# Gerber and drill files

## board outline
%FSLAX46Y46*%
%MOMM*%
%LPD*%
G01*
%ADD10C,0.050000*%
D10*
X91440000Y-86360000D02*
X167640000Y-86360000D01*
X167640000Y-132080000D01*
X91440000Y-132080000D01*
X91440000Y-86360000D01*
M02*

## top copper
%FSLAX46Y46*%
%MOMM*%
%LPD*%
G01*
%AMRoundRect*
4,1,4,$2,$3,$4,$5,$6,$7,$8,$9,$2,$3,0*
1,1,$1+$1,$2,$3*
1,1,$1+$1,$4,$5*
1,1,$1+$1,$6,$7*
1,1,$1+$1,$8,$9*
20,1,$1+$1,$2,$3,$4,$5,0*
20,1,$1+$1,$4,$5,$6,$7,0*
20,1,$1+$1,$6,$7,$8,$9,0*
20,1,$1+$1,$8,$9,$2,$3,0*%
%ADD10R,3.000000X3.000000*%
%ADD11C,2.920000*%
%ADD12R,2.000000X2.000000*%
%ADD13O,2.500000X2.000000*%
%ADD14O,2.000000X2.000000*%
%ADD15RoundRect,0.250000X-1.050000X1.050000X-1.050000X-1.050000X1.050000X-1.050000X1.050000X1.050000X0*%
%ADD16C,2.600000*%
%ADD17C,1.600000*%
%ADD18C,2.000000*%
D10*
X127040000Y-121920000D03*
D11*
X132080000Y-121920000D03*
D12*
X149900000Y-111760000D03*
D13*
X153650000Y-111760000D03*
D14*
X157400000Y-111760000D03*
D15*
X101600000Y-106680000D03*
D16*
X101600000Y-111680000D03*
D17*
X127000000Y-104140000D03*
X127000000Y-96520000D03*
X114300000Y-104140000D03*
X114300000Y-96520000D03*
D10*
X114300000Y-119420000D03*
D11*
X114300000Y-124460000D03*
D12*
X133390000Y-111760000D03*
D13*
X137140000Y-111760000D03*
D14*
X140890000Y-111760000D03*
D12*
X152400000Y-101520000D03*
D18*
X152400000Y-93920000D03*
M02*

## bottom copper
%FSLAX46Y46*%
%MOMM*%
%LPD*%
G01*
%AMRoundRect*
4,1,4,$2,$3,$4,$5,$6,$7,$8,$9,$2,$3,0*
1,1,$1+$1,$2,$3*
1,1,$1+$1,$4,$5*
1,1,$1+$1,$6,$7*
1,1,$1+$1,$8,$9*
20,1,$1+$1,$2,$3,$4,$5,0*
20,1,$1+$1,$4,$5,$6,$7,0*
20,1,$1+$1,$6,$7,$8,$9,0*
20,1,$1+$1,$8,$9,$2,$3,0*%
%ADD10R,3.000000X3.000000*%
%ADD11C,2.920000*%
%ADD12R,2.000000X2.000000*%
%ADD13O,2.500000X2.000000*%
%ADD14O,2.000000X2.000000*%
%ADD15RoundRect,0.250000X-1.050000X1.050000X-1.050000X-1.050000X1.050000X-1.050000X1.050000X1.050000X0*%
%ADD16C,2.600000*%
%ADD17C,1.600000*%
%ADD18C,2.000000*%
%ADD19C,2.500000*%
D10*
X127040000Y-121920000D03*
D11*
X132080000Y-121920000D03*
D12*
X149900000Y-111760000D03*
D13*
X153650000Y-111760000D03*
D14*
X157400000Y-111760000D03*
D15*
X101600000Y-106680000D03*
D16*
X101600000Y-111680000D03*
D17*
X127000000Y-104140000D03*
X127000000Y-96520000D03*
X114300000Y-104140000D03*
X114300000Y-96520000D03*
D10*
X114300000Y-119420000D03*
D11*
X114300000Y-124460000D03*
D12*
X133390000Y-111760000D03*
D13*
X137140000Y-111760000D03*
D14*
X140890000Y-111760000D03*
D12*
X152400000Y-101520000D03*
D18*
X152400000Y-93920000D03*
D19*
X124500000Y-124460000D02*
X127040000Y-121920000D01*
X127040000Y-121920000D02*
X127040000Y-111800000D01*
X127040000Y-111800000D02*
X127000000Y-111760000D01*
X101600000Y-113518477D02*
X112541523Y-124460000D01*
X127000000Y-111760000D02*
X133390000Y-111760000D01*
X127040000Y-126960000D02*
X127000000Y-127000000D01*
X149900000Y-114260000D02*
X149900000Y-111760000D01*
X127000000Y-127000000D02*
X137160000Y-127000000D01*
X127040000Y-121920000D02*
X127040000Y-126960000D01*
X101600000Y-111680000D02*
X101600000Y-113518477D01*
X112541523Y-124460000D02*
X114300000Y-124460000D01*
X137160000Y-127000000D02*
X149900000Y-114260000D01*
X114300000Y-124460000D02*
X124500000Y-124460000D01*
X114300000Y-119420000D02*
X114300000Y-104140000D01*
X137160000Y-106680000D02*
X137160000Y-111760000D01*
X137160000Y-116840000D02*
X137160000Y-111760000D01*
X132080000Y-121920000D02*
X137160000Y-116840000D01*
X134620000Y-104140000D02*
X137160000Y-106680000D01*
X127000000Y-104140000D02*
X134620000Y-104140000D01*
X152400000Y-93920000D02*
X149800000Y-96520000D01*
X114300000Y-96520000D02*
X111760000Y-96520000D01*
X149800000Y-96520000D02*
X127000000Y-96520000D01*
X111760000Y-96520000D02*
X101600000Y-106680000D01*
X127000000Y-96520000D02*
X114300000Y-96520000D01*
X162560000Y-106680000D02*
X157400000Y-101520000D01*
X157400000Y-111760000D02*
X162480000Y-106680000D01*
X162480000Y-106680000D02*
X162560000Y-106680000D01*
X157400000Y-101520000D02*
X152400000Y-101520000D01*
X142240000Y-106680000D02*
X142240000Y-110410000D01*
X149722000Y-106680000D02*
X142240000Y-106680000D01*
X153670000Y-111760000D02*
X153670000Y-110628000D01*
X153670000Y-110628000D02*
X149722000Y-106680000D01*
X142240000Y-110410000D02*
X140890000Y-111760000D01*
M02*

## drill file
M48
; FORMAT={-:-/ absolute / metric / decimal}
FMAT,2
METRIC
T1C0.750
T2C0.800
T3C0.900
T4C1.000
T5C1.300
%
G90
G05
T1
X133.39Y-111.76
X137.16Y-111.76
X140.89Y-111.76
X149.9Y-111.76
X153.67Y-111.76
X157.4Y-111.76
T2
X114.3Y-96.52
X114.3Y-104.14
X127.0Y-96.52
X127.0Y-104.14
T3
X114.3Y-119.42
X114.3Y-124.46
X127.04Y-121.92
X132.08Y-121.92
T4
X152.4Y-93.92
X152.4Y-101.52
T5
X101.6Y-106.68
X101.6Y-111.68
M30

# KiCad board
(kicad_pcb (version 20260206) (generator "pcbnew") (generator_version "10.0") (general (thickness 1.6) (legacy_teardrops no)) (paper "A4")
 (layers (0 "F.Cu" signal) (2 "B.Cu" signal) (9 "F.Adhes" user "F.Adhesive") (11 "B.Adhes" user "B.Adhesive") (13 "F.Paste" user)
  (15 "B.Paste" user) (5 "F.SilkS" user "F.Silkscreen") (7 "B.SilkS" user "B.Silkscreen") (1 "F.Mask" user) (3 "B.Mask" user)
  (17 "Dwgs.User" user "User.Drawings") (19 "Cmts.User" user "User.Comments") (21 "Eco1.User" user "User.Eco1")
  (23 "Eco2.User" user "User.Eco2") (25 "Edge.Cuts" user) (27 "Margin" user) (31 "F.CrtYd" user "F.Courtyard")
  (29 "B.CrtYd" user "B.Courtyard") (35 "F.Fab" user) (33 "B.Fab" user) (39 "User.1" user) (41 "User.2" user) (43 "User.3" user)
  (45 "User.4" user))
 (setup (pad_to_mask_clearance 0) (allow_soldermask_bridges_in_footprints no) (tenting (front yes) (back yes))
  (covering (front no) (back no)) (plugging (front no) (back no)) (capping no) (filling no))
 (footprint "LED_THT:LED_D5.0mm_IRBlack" (layer "F.Cu") (at 129.54 121.92)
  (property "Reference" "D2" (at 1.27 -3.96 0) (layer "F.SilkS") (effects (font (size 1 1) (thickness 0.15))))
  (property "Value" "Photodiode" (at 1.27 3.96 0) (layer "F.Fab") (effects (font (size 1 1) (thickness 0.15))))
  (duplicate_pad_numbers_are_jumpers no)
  (pad "1" thru_hole rect (at -2.5 0) (size 3 3) (drill 0.9) (layers "*.Cu" "*.Mask") (remove_unused_layers no) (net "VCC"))
  (pad "2" thru_hole circle (at 2.54 0) (size 2.92 2.92) (drill 0.9) (layers "*.Cu" "*.Mask") (remove_unused_layers no) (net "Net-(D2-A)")))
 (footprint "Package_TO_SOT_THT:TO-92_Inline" (layer "F.Cu") (at 152.4 111.76)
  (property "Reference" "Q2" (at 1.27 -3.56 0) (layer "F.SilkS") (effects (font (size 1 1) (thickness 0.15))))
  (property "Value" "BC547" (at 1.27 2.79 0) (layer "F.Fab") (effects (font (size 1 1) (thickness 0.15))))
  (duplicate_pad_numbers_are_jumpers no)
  (pad "1" thru_hole rect (at -2.5 0) (size 2 2) (drill 0.75) (layers "*.Cu" "*.Mask") (remove_unused_layers no) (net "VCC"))
  (pad "2" thru_hole oval (at 1.27 0) (size 2.5 2) (drill 0.75 (offset -0.02 0)) (layers "*.Cu" "*.Mask") (remove_unused_layers no)
   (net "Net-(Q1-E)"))
  (pad "3" thru_hole oval (at 5 0) (size 2 2) (drill 0.75) (layers "*.Cu" "*.Mask") (remove_unused_layers no) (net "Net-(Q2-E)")))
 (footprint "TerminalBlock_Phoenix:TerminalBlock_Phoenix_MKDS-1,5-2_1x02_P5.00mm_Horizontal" (layer "F.Cu") (at 101.6 106.68 -90)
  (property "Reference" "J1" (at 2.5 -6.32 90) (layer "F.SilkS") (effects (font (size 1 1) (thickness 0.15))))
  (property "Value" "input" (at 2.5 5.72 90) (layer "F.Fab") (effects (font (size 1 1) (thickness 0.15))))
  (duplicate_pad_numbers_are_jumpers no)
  (pad "1" thru_hole roundrect (at 0 0 270) (size 2.6 2.6) (drill 1.3) (layers "*.Cu" "*.Mask") (remove_unused_layers no)
   (roundrect_rratio 0.096154) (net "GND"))
  (pad "2" thru_hole circle (at 5 0 270) (size 2.6 2.6) (drill 1.3) (layers "*.Cu" "*.Mask") (remove_unused_layers no) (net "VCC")))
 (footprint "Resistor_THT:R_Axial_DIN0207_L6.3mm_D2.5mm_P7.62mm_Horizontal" (layer "F.Cu") (at 127 104.14 90)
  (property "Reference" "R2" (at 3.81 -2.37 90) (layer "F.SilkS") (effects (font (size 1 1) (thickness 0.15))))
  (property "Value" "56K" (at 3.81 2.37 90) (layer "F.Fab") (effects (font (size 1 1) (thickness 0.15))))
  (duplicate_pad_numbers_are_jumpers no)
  (pad "1" thru_hole circle (at 0 0 90) (size 1.6 1.6) (drill 0.8) (layers "*.Cu" "*.Mask") (remove_unused_layers no) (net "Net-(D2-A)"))
  (pad "2" thru_hole circle (at 7.62 0 90) (size 1.6 1.6) (drill 0.8) (layers "*.Cu" "*.Mask") (remove_unused_layers no) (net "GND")))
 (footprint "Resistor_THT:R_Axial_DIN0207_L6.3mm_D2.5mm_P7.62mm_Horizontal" (layer "F.Cu") (at 114.3 104.14 90)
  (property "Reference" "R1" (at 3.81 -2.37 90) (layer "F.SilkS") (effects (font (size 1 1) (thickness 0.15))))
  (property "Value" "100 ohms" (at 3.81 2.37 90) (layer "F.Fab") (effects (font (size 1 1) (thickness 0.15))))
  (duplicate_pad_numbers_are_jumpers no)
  (pad "1" thru_hole circle (at 0 0 90) (size 1.6 1.6) (drill 0.8) (layers "*.Cu" "*.Mask") (remove_unused_layers no) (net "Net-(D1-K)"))
  (pad "2" thru_hole circle (at 7.62 0 90) (size 1.6 1.6) (drill 0.8) (layers "*.Cu" "*.Mask") (remove_unused_layers no) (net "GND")))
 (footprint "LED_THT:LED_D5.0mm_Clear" (layer "F.Cu") (at 114.3 121.92 -90)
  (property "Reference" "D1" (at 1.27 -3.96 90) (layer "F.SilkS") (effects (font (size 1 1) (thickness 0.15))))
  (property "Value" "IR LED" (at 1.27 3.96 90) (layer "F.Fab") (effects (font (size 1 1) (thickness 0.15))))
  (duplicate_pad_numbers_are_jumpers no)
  (pad "1" thru_hole rect (at -2.5 0 270) (size 3 3) (drill 0.9) (layers "*.Cu" "*.Mask") (remove_unused_layers no) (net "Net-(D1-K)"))
  (pad "2" thru_hole circle (at 2.54 0 270) (size 2.92 2.92) (drill 0.9) (layers "*.Cu" "*.Mask") (remove_unused_layers no) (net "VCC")))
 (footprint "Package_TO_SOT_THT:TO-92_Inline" (layer "F.Cu") (at 135.89 111.76)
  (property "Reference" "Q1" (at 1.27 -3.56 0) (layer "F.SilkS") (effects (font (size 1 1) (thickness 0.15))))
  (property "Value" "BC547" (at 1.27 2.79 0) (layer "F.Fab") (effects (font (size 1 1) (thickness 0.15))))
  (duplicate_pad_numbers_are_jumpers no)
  (pad "1" thru_hole rect (at -2.5 0) (size 2 2) (drill 0.75) (layers "*.Cu" "*.Mask") (remove_unused_layers no) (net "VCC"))
  (pad "2" thru_hole oval (at 1.27 0) (size 2.5 2) (drill 0.75 (offset -0.02 0)) (layers "*.Cu" "*.Mask") (remove_unused_layers no)
   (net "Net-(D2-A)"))
  (pad "3" thru_hole oval (at 5 0) (size 2 2) (drill 0.75) (layers "*.Cu" "*.Mask") (remove_unused_layers no) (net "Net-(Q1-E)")))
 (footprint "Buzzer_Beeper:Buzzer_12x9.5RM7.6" (layer "F.Cu") (at 152.4 101.52 90)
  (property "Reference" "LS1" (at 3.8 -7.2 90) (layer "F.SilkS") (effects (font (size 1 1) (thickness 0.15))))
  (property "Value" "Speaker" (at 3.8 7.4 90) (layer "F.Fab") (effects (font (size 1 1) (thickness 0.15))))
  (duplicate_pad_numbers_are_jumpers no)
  (pad "1" thru_hole rect (at 0 0 90) (size 2 2) (drill 1) (layers "*.Cu" "*.Mask") (remove_unused_layers no) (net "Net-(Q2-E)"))
  (pad "2" thru_hole circle (at 7.6 0 90) (size 2 2) (drill 1) (layers "*.Cu" "*.Mask") (remove_unused_layers no) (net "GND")))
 (gr_rect (start 91.44 86.36) (end 167.64 132.08) (stroke (width 0.05) (type default)) (fill no) (layer "Edge.Cuts"))
 (segment (start 124.5 124.46) (end 127.04 121.92) (width 2.5) (layer "B.Cu") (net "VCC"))
 (segment (start 127.04 121.92) (end 127.04 111.8) (width 2.5) (layer "B.Cu") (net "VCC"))
 (segment (start 127.04 111.8) (end 127 111.76) (width 2.5) (layer "B.Cu") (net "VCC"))
 (segment (start 101.6 113.518477) (end 112.541523 124.46) (width 2.5) (layer "B.Cu") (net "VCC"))
 (segment (start 127 111.76) (end 133.39 111.76) (width 2.5) (layer "B.Cu") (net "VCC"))
 (segment (start 127.04 126.96) (end 127 127) (width 2.5) (layer "B.Cu") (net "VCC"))
 (segment (start 149.9 114.26) (end 149.9 111.76) (width 2.5) (layer "B.Cu") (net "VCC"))
 (segment (start 127 127) (end 137.16 127) (width 2.5) (layer "B.Cu") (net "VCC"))
 (segment (start 127.04 121.92) (end 127.04 126.96) (width 2.5) (layer "B.Cu") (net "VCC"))
 (segment (start 101.6 111.68) (end 101.6 113.518477) (width 2.5) (layer "B.Cu") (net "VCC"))
 (segment (start 112.541523 124.46) (end 114.3 124.46) (width 2.5) (layer "B.Cu") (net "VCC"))
 (segment (start 137.16 127) (end 149.9 114.26) (width 2.5) (layer "B.Cu") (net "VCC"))
 (segment (start 114.3 124.46) (end 124.5 124.46) (width 2.5) (layer "B.Cu") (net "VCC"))
 (segment (start 114.3 119.42) (end 114.3 104.14) (width 2.5) (layer "B.Cu") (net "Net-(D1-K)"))
 (segment (start 137.16 106.68) (end 137.16 111.76) (width 2.5) (layer "B.Cu") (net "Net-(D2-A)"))
 (segment (start 137.16 116.84) (end 137.16 111.76) (width 2.5) (layer "B.Cu") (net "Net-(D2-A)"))
 (segment (start 132.08 121.92) (end 137.16 116.84) (width 2.5) (layer "B.Cu") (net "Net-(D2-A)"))
 (segment (start 134.62 104.14) (end 137.16 106.68) (width 2.5) (layer "B.Cu") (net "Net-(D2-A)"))
 (segment (start 127 104.14) (end 134.62 104.14) (width 2.5) (layer "B.Cu") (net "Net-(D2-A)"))
 (segment (start 152.4 93.92) (end 149.8 96.52) (width 2.5) (layer "B.Cu") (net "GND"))
 (segment (start 114.3 96.52) (end 111.76 96.52) (width 2.5) (layer "B.Cu") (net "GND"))
 (segment (start 149.8 96.52) (end 127 96.52) (width 2.5) (layer "B.Cu") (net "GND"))
 (segment (start 111.76 96.52) (end 101.6 106.68) (width 2.5) (layer "B.Cu") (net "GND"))
 (segment (start 127 96.52) (end 114.3 96.52) (width 2.5) (layer "B.Cu") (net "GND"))
 (segment (start 162.56 106.68) (end 157.4 101.52) (width 2.5) (layer "B.Cu") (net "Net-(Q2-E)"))
 (segment (start 157.4 111.76) (end 162.48 106.68) (width 2.5) (layer "B.Cu") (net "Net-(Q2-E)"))
 (segment (start 162.48 106.68) (end 162.56 106.68) (width 2.5) (layer "B.Cu") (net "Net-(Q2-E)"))
 (segment (start 157.4 101.52) (end 152.4 101.52) (width 2.5) (layer "B.Cu") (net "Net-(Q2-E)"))
 (segment (start 142.24 106.68) (end 142.24 110.41) (width 2.5) (layer "B.Cu") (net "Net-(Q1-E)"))
 (segment (start 149.722 106.68) (end 142.24 106.68) (width 2.5) (layer "B.Cu") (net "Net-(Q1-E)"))
 (segment (start 153.67 111.76) (end 153.67 110.628) (width 2.5) (layer "B.Cu") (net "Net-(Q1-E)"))
 (segment (start 153.67 110.628) (end 149.722 106.68) (width 2.5) (layer "B.Cu") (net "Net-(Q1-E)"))
 (segment (start 142.24 110.41) (end 140.89 111.76) (width 2.5) (layer "B.Cu") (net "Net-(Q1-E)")))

